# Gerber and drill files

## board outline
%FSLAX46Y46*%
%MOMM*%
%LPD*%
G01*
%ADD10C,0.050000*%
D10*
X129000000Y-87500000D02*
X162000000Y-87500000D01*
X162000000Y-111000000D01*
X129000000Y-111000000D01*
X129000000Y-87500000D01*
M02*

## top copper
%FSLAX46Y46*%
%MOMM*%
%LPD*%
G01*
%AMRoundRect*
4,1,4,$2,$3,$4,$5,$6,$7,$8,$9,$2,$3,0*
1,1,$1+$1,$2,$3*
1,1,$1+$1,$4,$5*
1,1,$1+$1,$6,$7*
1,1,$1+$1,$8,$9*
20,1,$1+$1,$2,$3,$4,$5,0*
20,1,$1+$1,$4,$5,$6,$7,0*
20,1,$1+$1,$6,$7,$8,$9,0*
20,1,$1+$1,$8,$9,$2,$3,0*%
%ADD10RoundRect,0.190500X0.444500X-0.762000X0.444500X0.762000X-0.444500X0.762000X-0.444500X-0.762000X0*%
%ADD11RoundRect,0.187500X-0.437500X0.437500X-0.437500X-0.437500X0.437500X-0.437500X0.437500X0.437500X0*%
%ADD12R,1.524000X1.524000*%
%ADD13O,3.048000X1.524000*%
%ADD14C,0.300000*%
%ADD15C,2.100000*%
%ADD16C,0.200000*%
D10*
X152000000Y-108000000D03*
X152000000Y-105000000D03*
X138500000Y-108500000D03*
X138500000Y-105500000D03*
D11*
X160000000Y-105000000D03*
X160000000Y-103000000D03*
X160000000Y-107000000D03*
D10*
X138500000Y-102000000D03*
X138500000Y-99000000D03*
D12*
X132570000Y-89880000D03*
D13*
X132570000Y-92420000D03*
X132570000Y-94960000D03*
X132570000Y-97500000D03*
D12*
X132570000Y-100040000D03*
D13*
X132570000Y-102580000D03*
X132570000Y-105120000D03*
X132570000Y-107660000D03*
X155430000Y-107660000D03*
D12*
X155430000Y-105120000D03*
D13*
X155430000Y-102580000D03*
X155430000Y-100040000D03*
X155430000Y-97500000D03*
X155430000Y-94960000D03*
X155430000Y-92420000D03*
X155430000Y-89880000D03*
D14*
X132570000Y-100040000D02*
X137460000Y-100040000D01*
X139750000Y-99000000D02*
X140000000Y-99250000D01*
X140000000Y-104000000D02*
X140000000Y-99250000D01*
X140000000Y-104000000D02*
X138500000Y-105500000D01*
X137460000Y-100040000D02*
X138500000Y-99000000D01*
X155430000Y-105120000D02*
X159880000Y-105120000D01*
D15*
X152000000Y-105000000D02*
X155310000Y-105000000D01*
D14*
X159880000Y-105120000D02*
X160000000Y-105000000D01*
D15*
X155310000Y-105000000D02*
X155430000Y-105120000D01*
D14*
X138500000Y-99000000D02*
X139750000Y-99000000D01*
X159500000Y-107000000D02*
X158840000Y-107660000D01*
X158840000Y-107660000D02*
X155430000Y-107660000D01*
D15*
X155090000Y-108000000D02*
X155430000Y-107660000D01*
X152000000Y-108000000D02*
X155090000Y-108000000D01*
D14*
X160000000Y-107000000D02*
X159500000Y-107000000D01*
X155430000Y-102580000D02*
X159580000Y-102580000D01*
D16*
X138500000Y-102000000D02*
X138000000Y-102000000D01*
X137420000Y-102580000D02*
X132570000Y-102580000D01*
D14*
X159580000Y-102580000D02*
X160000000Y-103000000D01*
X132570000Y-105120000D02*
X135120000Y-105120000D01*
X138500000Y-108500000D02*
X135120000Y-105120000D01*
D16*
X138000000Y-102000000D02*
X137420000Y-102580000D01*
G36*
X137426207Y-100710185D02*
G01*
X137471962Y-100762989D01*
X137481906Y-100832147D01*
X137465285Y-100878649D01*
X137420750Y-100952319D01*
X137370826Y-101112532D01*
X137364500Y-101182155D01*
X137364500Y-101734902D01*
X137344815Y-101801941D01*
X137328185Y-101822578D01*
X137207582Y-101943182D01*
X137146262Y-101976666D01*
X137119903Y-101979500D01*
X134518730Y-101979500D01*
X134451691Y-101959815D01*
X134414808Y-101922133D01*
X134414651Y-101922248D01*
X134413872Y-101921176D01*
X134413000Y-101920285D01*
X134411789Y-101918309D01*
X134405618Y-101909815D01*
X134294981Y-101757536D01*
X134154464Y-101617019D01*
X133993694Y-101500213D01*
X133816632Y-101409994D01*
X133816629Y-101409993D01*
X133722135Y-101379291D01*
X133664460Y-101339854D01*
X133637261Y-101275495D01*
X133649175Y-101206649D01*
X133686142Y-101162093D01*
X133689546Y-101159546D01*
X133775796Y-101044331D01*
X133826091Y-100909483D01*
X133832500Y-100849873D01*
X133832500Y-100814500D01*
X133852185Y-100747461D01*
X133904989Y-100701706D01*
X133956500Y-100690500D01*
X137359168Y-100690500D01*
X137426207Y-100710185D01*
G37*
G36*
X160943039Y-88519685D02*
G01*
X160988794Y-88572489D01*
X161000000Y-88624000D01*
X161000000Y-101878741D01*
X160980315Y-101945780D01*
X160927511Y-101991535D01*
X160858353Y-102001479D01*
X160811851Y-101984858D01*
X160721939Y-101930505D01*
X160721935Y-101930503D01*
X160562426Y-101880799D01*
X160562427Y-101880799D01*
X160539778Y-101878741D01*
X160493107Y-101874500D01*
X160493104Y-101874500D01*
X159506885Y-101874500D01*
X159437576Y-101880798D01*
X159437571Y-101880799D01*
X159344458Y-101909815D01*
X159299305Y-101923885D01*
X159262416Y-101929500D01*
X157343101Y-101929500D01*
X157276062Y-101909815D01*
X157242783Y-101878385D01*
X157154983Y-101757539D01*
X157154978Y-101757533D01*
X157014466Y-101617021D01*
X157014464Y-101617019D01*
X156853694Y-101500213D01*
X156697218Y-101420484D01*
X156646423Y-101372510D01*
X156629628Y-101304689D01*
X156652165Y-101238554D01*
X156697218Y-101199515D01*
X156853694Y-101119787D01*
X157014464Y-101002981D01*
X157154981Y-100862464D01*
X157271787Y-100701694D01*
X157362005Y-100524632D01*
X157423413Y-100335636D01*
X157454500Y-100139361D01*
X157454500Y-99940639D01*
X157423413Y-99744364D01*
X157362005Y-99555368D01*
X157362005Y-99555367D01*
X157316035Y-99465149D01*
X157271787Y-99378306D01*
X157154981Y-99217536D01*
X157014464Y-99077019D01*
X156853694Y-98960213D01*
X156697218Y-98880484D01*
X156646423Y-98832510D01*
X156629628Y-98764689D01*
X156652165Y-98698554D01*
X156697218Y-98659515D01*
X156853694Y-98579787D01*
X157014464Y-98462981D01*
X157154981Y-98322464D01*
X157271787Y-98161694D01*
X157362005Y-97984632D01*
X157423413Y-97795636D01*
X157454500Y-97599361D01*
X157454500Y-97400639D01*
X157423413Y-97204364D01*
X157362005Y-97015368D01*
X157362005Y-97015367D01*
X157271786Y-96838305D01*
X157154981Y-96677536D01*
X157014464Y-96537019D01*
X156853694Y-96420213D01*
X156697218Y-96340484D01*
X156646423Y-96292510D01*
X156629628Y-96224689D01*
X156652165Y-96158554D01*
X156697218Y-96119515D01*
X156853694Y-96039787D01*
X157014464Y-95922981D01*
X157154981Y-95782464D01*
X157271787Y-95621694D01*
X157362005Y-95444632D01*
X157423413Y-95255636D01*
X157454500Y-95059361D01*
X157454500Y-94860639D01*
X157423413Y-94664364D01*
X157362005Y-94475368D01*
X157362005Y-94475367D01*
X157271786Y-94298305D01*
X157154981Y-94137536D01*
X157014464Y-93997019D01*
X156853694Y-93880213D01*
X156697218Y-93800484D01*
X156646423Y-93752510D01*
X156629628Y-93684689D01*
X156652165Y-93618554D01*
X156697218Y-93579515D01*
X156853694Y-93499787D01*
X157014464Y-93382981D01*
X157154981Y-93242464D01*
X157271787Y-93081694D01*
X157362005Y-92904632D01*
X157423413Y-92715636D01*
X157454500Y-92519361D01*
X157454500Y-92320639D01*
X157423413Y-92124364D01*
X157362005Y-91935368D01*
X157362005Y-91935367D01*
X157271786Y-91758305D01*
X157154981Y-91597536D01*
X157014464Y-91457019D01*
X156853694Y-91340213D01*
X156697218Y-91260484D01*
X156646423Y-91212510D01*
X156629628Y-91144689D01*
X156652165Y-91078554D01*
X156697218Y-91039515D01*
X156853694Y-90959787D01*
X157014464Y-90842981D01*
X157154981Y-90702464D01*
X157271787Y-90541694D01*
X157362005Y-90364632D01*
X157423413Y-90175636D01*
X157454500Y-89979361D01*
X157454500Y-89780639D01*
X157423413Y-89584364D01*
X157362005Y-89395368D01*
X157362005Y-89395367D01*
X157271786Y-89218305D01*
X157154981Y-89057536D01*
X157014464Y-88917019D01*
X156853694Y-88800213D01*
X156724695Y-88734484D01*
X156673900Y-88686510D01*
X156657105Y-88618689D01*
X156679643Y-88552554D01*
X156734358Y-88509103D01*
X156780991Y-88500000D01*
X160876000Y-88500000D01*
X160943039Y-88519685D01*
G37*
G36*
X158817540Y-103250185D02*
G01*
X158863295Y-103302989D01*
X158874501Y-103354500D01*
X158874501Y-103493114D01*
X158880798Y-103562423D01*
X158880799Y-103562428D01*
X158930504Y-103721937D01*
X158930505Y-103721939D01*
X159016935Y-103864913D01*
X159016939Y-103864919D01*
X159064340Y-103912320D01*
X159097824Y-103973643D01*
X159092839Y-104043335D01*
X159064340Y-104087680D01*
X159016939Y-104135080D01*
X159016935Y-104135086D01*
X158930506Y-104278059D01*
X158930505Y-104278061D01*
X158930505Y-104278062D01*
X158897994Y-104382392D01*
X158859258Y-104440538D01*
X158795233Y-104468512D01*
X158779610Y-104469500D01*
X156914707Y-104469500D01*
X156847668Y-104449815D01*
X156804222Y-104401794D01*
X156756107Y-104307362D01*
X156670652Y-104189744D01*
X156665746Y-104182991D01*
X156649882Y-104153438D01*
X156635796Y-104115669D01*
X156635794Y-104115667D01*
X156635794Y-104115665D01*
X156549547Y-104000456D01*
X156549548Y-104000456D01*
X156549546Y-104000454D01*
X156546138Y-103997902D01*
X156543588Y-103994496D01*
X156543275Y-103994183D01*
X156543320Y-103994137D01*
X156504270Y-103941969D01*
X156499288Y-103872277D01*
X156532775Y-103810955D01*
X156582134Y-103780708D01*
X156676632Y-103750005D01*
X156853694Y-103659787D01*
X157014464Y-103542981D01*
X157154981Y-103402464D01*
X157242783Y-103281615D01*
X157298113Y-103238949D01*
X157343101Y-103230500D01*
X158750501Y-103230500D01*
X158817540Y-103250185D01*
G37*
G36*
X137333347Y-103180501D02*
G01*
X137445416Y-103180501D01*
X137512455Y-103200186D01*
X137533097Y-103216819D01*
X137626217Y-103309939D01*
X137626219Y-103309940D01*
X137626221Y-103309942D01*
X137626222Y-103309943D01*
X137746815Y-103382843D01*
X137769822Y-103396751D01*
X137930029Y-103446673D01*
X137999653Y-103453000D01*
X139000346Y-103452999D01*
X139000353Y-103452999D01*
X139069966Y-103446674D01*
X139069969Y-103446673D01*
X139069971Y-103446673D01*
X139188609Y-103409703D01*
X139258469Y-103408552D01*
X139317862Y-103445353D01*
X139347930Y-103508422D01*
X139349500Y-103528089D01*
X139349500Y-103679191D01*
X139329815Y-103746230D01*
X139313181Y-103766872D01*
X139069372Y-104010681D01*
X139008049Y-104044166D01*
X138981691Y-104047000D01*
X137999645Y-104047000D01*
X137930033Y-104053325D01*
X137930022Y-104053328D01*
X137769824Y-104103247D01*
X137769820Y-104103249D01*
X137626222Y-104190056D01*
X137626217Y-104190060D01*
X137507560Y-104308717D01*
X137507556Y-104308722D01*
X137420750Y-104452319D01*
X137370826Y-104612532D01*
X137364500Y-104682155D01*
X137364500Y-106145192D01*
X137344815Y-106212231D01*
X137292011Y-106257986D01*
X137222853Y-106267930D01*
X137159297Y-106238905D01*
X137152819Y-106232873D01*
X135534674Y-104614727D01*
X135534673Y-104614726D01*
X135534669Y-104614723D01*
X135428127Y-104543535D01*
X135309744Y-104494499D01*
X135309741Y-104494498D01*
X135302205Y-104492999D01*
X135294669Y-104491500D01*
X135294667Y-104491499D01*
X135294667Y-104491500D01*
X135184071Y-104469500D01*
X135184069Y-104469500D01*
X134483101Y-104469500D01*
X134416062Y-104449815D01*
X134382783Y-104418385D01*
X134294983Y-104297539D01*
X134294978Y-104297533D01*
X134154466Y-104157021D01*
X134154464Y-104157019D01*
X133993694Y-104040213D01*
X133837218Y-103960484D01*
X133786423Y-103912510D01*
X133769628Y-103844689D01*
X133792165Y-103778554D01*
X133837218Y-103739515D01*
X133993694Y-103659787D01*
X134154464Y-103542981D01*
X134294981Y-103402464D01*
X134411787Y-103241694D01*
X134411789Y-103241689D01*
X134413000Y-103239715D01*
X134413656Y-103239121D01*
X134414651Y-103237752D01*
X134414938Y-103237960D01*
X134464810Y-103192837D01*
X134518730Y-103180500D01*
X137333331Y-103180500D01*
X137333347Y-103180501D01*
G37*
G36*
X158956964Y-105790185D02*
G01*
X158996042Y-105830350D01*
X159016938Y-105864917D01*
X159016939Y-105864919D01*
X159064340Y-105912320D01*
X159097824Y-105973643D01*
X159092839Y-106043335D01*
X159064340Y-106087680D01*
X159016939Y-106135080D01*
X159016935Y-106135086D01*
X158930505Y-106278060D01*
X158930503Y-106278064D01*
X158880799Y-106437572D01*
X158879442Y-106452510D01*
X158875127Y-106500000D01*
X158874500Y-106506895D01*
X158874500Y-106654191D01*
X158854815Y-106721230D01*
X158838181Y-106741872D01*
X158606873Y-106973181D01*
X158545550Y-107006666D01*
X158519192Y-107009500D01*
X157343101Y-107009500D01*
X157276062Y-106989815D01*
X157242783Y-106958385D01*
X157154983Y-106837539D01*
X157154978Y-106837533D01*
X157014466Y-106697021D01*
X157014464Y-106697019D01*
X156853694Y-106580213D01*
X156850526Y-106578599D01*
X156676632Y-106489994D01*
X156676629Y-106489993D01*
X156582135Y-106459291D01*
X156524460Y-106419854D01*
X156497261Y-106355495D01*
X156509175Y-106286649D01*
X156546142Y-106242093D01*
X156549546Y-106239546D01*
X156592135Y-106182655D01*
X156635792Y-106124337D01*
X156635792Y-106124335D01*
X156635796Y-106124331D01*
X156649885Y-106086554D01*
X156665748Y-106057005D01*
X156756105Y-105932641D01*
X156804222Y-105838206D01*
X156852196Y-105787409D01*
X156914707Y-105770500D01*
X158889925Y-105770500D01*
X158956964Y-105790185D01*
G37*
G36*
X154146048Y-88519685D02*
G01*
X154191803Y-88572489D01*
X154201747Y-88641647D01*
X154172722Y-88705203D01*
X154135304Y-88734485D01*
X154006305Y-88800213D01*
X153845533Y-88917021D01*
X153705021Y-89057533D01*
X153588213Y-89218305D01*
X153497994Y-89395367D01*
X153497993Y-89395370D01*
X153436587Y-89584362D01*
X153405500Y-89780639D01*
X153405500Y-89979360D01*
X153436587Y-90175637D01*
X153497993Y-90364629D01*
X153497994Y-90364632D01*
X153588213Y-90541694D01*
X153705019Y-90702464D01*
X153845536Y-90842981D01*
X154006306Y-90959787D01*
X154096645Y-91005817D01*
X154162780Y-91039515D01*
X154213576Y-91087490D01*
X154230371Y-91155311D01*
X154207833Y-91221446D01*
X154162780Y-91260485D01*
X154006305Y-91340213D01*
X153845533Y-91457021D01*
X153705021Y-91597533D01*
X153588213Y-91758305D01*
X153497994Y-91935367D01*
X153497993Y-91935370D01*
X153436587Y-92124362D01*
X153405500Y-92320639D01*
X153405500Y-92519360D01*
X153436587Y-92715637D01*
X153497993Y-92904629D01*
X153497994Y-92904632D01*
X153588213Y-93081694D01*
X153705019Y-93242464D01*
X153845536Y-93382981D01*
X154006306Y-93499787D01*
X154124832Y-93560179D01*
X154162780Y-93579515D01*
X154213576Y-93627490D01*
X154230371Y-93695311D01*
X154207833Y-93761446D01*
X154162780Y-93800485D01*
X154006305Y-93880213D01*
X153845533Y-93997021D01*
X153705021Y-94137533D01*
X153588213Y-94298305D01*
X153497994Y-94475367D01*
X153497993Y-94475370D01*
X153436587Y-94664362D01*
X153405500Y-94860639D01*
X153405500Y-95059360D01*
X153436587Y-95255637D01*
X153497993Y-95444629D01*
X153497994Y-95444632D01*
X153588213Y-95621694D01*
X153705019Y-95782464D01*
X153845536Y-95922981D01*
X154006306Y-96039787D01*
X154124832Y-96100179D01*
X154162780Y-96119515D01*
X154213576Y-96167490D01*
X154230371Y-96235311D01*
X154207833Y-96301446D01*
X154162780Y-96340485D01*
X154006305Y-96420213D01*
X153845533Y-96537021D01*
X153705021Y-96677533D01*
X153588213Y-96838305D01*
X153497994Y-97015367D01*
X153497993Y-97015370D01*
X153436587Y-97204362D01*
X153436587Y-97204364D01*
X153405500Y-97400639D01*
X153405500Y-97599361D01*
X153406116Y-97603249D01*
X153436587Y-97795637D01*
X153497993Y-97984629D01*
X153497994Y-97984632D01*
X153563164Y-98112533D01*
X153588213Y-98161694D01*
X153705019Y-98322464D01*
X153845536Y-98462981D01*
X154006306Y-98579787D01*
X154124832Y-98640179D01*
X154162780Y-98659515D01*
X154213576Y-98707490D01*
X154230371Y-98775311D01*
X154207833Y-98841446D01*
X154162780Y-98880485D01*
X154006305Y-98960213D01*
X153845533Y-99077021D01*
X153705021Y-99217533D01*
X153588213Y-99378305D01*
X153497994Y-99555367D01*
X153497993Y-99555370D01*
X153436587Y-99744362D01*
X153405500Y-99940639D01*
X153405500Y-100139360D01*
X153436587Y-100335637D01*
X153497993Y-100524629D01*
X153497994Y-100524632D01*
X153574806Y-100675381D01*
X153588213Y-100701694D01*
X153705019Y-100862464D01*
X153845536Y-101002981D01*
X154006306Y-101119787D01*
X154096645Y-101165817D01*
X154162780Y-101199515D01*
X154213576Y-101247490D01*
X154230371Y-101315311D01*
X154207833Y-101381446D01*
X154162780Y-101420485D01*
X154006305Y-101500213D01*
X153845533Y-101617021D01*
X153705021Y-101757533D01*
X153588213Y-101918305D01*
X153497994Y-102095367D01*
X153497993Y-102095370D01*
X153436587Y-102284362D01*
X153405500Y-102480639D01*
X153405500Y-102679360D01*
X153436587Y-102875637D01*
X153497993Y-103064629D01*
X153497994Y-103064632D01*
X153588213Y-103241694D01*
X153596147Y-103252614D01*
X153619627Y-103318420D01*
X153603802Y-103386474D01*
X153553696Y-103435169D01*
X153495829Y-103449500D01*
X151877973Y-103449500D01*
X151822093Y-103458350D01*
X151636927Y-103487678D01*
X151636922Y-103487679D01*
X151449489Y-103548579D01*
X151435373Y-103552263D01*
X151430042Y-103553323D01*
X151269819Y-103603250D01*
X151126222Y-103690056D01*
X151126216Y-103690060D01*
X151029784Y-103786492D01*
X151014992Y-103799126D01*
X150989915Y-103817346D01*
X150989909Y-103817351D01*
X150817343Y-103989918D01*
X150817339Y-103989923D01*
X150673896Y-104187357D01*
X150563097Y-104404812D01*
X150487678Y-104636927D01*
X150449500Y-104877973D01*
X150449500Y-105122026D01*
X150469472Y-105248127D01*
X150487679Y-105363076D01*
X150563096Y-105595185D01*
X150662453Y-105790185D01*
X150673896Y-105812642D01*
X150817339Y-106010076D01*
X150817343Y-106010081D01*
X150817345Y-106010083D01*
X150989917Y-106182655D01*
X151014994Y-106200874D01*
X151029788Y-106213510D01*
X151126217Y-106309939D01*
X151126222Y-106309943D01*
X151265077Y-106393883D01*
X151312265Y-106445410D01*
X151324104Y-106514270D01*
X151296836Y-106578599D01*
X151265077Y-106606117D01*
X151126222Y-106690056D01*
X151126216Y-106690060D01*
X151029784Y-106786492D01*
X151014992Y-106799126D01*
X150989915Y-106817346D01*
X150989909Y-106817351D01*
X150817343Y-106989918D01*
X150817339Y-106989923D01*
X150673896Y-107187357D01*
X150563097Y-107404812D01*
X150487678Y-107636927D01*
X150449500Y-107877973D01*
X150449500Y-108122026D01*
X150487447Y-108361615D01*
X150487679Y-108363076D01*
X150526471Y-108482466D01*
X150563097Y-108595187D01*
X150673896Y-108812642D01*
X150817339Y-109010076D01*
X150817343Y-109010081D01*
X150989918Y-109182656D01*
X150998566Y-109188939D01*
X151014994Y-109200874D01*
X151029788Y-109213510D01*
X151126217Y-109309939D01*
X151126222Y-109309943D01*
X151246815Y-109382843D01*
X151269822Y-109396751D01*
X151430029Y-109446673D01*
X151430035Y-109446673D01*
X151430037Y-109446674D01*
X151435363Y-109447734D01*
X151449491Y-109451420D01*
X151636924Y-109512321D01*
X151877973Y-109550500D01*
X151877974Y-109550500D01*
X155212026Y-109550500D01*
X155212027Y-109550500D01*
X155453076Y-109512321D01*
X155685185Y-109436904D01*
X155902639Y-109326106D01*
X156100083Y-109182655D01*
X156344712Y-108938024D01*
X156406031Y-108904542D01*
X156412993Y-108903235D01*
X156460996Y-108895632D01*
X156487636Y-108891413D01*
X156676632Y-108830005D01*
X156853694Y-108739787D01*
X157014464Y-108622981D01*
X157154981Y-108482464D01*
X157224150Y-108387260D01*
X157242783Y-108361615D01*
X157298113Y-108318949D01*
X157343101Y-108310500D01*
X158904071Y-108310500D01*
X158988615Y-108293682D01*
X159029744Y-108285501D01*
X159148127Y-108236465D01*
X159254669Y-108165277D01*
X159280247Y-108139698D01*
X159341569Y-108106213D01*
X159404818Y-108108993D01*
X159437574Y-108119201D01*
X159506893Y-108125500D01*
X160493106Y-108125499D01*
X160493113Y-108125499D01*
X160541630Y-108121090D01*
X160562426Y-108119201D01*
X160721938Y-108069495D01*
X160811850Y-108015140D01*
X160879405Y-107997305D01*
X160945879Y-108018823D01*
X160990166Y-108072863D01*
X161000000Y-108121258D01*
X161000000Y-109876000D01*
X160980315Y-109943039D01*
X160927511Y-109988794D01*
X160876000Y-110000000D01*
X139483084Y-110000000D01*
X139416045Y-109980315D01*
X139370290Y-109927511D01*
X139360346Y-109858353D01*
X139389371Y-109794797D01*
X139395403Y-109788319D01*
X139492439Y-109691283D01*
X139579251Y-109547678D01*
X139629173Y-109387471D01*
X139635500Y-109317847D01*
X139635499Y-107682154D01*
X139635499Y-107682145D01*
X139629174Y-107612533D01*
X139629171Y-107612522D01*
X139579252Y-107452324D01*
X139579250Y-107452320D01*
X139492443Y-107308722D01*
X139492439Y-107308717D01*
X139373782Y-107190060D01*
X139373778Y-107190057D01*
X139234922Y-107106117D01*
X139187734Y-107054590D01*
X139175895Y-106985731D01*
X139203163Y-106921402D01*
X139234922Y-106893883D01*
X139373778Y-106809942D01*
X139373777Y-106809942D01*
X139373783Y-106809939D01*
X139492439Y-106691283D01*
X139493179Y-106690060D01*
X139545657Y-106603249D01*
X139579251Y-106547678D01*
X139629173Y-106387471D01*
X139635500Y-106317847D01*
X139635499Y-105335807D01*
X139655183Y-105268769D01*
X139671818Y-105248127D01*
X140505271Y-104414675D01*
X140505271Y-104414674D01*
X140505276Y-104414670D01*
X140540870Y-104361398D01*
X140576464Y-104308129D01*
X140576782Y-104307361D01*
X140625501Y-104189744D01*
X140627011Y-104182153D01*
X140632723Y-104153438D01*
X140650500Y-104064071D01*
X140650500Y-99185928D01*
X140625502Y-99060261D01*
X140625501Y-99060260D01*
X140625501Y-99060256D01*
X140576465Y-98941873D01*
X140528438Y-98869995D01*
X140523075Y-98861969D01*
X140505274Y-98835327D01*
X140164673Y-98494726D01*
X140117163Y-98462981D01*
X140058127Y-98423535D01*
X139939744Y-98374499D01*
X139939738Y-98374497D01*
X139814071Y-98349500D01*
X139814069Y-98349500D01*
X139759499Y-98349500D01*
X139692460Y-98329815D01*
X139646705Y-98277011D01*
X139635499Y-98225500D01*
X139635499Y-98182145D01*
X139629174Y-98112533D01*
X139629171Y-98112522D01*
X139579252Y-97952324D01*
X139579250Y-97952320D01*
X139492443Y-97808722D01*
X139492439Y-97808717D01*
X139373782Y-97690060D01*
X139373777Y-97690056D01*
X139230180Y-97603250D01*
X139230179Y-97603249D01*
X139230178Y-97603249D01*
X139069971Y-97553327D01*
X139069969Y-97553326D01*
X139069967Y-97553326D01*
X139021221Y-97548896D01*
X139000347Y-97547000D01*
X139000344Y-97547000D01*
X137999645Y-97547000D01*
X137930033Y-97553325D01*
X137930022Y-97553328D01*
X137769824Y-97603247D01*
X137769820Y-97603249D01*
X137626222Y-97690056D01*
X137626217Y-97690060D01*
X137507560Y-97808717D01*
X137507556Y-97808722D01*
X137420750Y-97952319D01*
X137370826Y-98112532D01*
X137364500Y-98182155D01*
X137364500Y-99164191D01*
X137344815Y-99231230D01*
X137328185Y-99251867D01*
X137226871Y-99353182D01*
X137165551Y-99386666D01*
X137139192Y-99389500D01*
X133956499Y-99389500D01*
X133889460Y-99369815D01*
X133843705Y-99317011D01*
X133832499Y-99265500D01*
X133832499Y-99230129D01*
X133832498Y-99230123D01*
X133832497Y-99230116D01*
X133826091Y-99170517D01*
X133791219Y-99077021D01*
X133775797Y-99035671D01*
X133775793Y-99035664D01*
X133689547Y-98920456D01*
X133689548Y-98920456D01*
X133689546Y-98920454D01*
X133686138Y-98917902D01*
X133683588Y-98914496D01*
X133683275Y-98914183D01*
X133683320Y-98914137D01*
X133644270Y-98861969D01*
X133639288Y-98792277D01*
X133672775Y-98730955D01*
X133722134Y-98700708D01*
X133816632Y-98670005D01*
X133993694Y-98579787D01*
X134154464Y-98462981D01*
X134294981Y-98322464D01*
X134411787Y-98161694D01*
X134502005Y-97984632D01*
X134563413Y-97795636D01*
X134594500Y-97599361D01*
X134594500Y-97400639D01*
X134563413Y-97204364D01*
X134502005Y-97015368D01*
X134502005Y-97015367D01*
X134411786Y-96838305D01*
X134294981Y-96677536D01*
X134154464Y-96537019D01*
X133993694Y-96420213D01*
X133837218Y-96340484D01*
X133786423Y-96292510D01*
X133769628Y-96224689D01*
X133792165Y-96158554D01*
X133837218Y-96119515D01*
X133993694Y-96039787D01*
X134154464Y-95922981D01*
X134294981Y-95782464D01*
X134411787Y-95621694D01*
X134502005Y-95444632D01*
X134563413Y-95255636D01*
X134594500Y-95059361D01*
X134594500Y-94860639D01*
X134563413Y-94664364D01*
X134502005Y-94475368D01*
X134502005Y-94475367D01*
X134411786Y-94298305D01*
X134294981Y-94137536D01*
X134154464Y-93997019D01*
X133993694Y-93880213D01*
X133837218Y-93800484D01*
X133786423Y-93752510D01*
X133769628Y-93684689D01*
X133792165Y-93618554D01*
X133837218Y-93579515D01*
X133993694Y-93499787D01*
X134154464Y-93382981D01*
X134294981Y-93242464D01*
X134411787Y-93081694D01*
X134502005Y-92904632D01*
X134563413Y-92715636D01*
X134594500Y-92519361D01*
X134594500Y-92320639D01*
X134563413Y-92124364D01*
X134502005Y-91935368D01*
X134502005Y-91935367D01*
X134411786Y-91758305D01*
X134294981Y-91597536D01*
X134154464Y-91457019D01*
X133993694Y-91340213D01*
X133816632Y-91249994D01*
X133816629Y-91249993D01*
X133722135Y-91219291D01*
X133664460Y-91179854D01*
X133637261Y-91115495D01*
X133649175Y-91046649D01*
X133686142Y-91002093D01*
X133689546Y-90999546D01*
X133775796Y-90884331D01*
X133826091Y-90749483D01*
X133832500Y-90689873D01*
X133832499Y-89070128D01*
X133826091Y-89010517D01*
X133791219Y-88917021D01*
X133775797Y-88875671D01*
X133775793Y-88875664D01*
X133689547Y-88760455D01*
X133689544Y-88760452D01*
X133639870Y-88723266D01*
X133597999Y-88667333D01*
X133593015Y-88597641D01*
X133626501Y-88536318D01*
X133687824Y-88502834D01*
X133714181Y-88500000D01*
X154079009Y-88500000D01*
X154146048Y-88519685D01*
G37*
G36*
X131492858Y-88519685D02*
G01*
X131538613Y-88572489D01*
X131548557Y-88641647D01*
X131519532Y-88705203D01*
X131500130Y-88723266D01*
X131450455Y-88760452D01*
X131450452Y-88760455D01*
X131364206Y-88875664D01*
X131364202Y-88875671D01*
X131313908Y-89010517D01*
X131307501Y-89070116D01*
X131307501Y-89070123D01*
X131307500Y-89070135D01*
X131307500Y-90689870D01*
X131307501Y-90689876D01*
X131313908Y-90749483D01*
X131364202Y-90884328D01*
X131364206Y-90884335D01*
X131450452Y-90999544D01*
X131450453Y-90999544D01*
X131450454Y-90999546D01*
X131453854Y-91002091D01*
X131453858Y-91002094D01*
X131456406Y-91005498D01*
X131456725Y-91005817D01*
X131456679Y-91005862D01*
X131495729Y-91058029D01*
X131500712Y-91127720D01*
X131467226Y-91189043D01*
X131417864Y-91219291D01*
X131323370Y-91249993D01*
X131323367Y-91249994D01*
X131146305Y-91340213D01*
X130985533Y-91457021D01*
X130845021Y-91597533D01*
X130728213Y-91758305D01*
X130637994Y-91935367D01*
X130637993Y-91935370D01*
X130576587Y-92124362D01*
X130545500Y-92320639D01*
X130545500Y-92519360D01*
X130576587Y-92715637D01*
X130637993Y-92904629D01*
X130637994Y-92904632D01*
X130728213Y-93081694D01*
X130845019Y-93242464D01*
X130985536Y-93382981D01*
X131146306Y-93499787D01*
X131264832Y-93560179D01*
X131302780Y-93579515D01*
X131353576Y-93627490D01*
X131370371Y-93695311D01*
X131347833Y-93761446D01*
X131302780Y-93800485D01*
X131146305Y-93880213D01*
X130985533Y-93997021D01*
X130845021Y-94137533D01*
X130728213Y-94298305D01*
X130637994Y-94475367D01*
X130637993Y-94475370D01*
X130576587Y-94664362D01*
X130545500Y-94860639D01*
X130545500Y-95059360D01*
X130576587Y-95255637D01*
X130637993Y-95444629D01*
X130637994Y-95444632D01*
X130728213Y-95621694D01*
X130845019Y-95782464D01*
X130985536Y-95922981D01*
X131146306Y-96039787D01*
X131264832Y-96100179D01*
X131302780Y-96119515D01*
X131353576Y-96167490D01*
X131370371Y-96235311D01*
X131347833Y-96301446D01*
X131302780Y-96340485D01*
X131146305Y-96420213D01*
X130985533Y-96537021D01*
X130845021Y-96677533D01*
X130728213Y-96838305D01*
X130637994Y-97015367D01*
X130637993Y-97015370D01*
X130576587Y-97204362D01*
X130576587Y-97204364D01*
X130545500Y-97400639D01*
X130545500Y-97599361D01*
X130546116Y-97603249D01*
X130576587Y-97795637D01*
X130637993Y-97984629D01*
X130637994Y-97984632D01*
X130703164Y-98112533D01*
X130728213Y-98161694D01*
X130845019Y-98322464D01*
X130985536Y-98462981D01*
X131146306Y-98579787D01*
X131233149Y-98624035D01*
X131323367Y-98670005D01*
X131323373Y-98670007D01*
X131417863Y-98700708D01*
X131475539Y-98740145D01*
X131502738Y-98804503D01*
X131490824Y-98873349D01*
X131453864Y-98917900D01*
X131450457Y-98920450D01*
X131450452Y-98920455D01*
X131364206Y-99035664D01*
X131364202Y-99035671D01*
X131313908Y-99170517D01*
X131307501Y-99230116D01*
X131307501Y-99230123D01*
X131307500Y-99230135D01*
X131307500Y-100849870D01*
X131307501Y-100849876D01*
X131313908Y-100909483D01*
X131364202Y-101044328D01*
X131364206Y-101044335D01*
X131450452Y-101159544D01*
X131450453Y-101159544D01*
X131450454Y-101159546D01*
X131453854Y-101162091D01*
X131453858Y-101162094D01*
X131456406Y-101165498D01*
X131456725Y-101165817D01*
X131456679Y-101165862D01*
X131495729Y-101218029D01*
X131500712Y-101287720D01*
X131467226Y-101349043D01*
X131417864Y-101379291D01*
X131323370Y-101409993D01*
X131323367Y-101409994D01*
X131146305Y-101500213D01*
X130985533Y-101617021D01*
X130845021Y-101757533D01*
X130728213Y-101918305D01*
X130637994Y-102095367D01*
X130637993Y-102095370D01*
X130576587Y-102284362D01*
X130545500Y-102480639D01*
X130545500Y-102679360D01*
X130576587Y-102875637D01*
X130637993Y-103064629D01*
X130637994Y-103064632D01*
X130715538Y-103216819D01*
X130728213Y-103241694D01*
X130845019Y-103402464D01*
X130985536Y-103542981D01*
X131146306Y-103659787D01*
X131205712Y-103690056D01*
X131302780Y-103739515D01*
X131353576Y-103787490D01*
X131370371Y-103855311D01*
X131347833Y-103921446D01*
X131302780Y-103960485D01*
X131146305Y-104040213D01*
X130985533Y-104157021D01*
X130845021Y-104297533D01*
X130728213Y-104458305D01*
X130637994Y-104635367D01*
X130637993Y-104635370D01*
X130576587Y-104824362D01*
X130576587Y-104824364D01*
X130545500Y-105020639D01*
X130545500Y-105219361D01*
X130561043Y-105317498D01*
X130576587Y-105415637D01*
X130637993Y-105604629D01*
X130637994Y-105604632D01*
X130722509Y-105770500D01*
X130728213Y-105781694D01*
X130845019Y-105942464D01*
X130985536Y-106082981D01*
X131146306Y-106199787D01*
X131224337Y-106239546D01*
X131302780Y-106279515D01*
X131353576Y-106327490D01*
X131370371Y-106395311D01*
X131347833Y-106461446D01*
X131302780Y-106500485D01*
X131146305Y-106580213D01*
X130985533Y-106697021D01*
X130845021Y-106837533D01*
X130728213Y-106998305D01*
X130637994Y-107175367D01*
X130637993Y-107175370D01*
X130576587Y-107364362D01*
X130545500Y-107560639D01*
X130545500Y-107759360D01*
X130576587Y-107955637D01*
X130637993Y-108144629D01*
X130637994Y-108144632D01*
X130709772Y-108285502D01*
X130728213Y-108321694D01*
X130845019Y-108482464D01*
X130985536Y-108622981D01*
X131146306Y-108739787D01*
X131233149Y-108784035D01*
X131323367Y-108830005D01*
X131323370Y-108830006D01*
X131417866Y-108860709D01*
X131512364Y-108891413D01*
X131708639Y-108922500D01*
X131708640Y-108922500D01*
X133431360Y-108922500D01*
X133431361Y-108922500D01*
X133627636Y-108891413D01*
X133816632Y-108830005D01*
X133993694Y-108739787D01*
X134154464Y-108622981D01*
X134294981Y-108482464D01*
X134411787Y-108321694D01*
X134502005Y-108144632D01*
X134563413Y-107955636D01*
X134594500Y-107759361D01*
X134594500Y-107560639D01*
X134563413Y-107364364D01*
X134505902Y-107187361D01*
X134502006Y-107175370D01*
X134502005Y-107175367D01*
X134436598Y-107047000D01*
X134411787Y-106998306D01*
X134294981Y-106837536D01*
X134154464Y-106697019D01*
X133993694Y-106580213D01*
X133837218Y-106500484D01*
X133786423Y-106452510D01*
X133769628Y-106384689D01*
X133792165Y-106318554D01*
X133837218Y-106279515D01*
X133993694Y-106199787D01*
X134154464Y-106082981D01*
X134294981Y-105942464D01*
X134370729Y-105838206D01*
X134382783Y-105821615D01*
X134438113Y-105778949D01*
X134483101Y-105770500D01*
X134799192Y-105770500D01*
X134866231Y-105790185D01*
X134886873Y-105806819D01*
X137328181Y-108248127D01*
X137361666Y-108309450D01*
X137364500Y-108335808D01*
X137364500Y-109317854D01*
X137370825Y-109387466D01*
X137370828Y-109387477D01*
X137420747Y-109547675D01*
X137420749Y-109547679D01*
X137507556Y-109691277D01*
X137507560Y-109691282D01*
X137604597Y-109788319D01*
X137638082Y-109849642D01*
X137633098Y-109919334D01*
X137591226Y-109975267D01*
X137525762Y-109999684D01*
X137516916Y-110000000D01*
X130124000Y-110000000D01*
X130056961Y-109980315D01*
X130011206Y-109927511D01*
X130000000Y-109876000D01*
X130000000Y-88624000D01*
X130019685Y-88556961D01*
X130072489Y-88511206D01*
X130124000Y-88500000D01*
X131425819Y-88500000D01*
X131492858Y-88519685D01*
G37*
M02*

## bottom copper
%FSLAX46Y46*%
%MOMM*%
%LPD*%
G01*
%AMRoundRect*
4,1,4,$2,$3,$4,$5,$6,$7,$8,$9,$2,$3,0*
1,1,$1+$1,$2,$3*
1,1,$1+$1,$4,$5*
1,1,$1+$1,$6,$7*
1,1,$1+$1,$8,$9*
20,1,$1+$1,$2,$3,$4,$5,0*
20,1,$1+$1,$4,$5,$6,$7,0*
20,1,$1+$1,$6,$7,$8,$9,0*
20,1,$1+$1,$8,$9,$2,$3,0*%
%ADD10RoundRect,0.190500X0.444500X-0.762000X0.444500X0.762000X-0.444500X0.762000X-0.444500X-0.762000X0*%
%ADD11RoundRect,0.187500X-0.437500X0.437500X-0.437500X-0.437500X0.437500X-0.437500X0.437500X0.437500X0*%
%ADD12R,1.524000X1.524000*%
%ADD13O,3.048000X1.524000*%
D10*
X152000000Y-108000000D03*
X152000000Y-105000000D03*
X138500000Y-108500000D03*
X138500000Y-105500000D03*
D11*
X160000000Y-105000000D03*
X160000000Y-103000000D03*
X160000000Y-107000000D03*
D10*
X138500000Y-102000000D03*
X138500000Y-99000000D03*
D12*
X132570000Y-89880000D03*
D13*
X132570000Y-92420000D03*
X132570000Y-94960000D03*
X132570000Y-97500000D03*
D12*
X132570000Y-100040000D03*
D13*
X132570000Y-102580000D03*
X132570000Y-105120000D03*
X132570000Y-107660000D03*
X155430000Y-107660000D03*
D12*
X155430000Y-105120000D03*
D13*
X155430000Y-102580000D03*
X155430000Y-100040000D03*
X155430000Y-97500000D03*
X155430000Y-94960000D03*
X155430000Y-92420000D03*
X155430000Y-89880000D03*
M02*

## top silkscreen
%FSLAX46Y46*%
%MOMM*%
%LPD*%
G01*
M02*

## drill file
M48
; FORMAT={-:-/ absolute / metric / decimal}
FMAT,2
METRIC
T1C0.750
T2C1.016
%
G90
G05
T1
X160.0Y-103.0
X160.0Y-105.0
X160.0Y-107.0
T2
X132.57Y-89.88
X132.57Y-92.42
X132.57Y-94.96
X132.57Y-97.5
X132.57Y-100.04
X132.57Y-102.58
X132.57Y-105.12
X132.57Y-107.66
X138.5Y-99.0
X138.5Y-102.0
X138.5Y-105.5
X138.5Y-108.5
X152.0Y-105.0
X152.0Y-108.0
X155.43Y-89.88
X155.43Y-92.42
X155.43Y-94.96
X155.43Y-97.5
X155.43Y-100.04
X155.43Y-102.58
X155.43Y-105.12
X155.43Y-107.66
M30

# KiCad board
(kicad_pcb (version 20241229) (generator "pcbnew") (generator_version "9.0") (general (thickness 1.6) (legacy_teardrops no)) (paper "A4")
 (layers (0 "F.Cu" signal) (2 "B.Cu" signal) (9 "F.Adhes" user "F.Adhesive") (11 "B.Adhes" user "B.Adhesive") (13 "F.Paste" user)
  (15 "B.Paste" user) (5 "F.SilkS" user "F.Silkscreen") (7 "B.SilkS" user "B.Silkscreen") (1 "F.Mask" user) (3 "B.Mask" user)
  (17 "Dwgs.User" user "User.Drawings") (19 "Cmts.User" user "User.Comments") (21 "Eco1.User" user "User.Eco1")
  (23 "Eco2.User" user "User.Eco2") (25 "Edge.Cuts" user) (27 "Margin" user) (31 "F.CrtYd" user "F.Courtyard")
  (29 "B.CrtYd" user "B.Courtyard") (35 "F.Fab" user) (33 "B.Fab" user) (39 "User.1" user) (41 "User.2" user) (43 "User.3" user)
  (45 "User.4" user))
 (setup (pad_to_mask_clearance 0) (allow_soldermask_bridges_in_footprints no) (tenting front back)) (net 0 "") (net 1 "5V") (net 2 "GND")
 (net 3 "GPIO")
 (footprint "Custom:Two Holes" (layer "F.Cu") (at 147.5 106.5 90)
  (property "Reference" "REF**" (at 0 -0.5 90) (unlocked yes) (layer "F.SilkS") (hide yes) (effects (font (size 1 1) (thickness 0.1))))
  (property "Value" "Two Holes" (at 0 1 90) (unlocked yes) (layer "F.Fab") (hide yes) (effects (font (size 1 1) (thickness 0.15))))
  (pad "1" thru_hole roundrect (at -1.5 4.5 90) (size 1.905 1.27) (drill 1.016) (layers "*.Cu" "*.Mask") (remove_unused_layers no)
   (roundrect_rratio 0.15) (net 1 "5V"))
  (pad "2" thru_hole roundrect (at 1.5 4.5 90) (size 1.905 1.27) (drill 1.016) (layers "*.Cu" "*.Mask") (remove_unused_layers no)
   (roundrect_rratio 0.15) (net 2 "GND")))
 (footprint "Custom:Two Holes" (layer "F.Cu") (at 134 107 90)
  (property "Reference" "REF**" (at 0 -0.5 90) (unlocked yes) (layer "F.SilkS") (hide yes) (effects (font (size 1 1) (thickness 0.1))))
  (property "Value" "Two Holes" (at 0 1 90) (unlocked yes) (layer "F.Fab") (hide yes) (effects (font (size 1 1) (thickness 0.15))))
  (pad "1" thru_hole roundrect (at -1.5 4.5 90) (size 1.905 1.27) (drill 1.016) (layers "*.Cu" "*.Mask") (remove_unused_layers no)
   (roundrect_rratio 0.15) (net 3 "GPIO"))
  (pad "2" thru_hole roundrect (at 1.5 4.5 90) (size 1.905 1.27) (drill 1.016) (layers "*.Cu" "*.Mask") (remove_unused_layers no)
   (roundrect_rratio 0.15) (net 2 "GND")))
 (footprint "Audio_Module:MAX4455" (layer "F.Cu") (at 160 105 -90)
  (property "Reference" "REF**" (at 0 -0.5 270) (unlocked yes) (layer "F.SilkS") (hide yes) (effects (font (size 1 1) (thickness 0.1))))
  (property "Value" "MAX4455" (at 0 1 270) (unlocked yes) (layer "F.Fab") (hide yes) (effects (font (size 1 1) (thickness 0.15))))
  (pad "GND" thru_hole roundrect (at 0 0 270) (size 1.25 1.25) (drill 0.75) (layers "*.Cu" "*.Mask") (remove_unused_layers no)
   (roundrect_rratio 0.15) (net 2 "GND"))
  (pad "OUT" thru_hole roundrect (at -2 0 270) (size 1.25 1.25) (drill 0.75) (layers "*.Cu" "*.Mask") (remove_unused_layers no)
   (roundrect_rratio 0.15) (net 3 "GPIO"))
  (pad "VCC" thru_hole roundrect (at 2 0 270) (size 1.25 1.25) (drill 0.75) (layers "*.Cu" "*.Mask") (remove_unused_layers no)
   (roundrect_rratio 0.15) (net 1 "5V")))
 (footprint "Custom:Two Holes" (layer "F.Cu") (at 134 100.5 90)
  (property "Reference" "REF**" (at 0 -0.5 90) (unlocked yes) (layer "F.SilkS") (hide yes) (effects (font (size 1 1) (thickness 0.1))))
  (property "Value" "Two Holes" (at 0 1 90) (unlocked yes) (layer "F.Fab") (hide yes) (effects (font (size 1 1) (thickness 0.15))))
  (pad "1" thru_hole roundrect (at -1.5 4.5 90) (size 1.905 1.27) (drill 1.016) (layers "*.Cu" "*.Mask") (remove_unused_layers no)
   (roundrect_rratio 0.15) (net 3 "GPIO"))
  (pad "2" thru_hole roundrect (at 1.5 4.5 90) (size 1.905 1.27) (drill 1.016) (layers "*.Cu" "*.Mask") (remove_unused_layers no)
   (roundrect_rratio 0.15) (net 2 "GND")))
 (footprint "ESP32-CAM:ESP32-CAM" (layer "F.Cu") (at 144 97.5)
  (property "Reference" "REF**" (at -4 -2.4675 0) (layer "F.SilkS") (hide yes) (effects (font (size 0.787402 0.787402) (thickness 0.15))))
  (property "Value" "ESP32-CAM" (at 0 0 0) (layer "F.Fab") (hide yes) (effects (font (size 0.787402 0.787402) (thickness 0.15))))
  (pad "P$1" thru_hole rect (at -11.43 -7.62) (size 1.524 1.524) (drill 1.016) (layers "*.Cu" "*.Mask") (remove_unused_layers no)
   (solder_mask_margin 0.102))
  (pad "P$2" thru_hole oval (at -11.43 -5.08) (size 3.048 1.524) (drill 1.016) (layers "*.Cu" "*.Mask") (remove_unused_layers no)
   (solder_mask_margin 0.102))
  (pad "P$3" thru_hole oval (at -11.43 -2.54) (size 3.048 1.524) (drill 1.016) (layers "*.Cu" "*.Mask") (remove_unused_layers no)
   (solder_mask_margin 0.102))
  (pad "P$4" thru_hole oval (at -11.43 0) (size 3.048 1.524) (drill 1.016) (layers "*.Cu" "*.Mask") (remove_unused_layers no)
   (solder_mask_margin 0.102))
  (pad "P$5" thru_hole rect (at -11.43 2.54) (size 1.524 1.524) (drill 1.016) (layers "*.Cu" "*.Mask") (remove_unused_layers no)
   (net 2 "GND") (solder_mask_margin 0.102))
  (pad "P$6" thru_hole oval (at -11.43 5.08) (size 3.048 1.524) (drill 1.016) (layers "*.Cu" "*.Mask") (remove_unused_layers no)
   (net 3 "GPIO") (solder_mask_margin 0.102))
  (pad "P$7" thru_hole oval (at -11.43 7.62) (size 3.048 1.524) (drill 1.016) (layers "*.Cu" "*.Mask") (remove_unused_layers no)
   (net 3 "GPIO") (solder_mask_margin 0.102))
  (pad "P$8" thru_hole oval (at -11.43 10.16) (size 3.048 1.524) (drill 1.016) (layers "*.Cu" "*.Mask") (remove_unused_layers no)
   (solder_mask_margin 0.102))
  (pad "P$9" thru_hole oval (at 11.43 10.16) (size 3.048 1.524) (drill 1.016) (layers "*.Cu" "*.Mask") (remove_unused_layers no)
   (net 1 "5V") (solder_mask_margin 0.102))
  (pad "P$10" thru_hole rect (at 11.43 7.62) (size 1.524 1.524) (drill 1.016) (layers "*.Cu" "*.Mask") (remove_unused_layers no)
   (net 2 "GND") (solder_mask_margin 0.102))
  (pad "P$11" thru_hole oval (at 11.43 5.08) (size 3.048 1.524) (drill 1.016) (layers "*.Cu" "*.Mask") (remove_unused_layers no)
   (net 3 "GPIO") (solder_mask_margin 0.102))
  (pad "P$12" thru_hole oval (at 11.43 2.54) (size 3.048 1.524) (drill 1.016) (layers "*.Cu" "*.Mask") (remove_unused_layers no)
   (solder_mask_margin 0.102))
  (pad "P$13" thru_hole oval (at 11.43 0) (size 3.048 1.524) (drill 1.016) (layers "*.Cu" "*.Mask") (remove_unused_layers no)
   (solder_mask_margin 0.102))
  (pad "P$14" thru_hole oval (at 11.43 -2.54) (size 3.048 1.524) (drill 1.016) (layers "*.Cu" "*.Mask") (remove_unused_layers no)
   (solder_mask_margin 0.102))
  (pad "P$15" thru_hole oval (at 11.43 -5.08) (size 3.048 1.524) (drill 1.016) (layers "*.Cu" "*.Mask") (remove_unused_layers no)
   (solder_mask_margin 0.102))
  (pad "P$16" thru_hole oval (at 11.43 -7.62) (size 3.048 1.524) (drill 1.016) (layers "*.Cu" "*.Mask") (remove_unused_layers no)
   (solder_mask_margin 0.102)))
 (gr_rect (start 129 87.5) (end 162 111) (stroke (width 0.05) (type default)) (fill no) (layer "Edge.Cuts"))
 (segment (start 132.57 100.04) (end 137.46 100.04) (width 0.3) (layers "F.Cu" "F.Mask") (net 2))
 (segment (start 139.75 99) (end 140 99.25) (width 0.3) (layers "F.Cu" "F.Mask") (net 2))
 (segment (start 140 104) (end 140 99.25) (width 0.3) (layers "F.Cu" "F.Mask") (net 2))
 (segment (start 140 104) (end 138.5 105.5) (width 0.3) (layers "F.Cu" "F.Mask") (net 2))
 (segment (start 137.46 100.04) (end 138.5 99) (width 0.3) (layers "F.Cu" "F.Mask") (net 2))
 (segment (start 155.43 105.12) (end 159.88 105.12) (width 0.3) (layers "F.Cu" "F.Mask") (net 2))
 (segment (start 152 105) (end 155.31 105) (width 2.1) (layers "F.Cu" "F.Mask") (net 2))
 (segment (start 159.88 105.12) (end 160 105) (width 0.3) (layer "F.Cu") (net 2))
 (segment (start 155.31 105) (end 155.43 105.12) (width 2.1) (layers "F.Cu" "F.Mask") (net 2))
 (segment (start 138.5 99) (end 139.75 99) (width 0.3) (layers "F.Cu" "F.Mask") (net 2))
 (segment (start 159.5 107) (end 158.84 107.66) (width 0.3) (layers "F.Cu" "F.Mask") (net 1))
 (segment (start 158.84 107.66) (end 155.43 107.66) (width 0.3) (layers "F.Cu" "F.Mask") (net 1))
 (segment (start 155.09 108) (end 155.43 107.66) (width 2.1) (layers "F.Cu" "F.Mask") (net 1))
 (segment (start 152 108) (end 155.09 108) (width 2.1) (layers "F.Cu" "F.Mask") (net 1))
 (segment (start 160 107) (end 159.5 107) (width 0.3) (layer "F.Cu") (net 1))
 (segment (start 155.43 102.58) (end 159.58 102.58) (width 0.3) (layers "F.Cu" "F.Mask") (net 3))
 (segment (start 138.5 102) (end 138 102) (width 0.2) (layer "F.Cu") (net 3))
 (segment (start 137.42 102.58) (end 132.57 102.58) (width 0.2) (layers "F.Cu" "F.Mask") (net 3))
 (segment (start 159.58 102.58) (end 160 103) (width 0.3) (layer "F.Cu") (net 3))
 (segment (start 132.57 105.12) (end 135.12 105.12) (width 0.3) (layers "F.Cu" "F.Mask") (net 3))
 (segment (start 138.5 108.5) (end 135.12 105.12) (width 0.3) (layers "F.Cu" "F.Mask") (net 3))
 (segment (start 138 102) (end 137.42 102.58) (width 0.2) (layers "F.Cu" "F.Mask") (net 3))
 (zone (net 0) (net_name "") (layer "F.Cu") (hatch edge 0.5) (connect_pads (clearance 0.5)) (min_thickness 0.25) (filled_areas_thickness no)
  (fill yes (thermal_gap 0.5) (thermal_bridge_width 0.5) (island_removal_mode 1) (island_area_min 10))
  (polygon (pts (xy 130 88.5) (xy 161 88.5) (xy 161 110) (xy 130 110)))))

